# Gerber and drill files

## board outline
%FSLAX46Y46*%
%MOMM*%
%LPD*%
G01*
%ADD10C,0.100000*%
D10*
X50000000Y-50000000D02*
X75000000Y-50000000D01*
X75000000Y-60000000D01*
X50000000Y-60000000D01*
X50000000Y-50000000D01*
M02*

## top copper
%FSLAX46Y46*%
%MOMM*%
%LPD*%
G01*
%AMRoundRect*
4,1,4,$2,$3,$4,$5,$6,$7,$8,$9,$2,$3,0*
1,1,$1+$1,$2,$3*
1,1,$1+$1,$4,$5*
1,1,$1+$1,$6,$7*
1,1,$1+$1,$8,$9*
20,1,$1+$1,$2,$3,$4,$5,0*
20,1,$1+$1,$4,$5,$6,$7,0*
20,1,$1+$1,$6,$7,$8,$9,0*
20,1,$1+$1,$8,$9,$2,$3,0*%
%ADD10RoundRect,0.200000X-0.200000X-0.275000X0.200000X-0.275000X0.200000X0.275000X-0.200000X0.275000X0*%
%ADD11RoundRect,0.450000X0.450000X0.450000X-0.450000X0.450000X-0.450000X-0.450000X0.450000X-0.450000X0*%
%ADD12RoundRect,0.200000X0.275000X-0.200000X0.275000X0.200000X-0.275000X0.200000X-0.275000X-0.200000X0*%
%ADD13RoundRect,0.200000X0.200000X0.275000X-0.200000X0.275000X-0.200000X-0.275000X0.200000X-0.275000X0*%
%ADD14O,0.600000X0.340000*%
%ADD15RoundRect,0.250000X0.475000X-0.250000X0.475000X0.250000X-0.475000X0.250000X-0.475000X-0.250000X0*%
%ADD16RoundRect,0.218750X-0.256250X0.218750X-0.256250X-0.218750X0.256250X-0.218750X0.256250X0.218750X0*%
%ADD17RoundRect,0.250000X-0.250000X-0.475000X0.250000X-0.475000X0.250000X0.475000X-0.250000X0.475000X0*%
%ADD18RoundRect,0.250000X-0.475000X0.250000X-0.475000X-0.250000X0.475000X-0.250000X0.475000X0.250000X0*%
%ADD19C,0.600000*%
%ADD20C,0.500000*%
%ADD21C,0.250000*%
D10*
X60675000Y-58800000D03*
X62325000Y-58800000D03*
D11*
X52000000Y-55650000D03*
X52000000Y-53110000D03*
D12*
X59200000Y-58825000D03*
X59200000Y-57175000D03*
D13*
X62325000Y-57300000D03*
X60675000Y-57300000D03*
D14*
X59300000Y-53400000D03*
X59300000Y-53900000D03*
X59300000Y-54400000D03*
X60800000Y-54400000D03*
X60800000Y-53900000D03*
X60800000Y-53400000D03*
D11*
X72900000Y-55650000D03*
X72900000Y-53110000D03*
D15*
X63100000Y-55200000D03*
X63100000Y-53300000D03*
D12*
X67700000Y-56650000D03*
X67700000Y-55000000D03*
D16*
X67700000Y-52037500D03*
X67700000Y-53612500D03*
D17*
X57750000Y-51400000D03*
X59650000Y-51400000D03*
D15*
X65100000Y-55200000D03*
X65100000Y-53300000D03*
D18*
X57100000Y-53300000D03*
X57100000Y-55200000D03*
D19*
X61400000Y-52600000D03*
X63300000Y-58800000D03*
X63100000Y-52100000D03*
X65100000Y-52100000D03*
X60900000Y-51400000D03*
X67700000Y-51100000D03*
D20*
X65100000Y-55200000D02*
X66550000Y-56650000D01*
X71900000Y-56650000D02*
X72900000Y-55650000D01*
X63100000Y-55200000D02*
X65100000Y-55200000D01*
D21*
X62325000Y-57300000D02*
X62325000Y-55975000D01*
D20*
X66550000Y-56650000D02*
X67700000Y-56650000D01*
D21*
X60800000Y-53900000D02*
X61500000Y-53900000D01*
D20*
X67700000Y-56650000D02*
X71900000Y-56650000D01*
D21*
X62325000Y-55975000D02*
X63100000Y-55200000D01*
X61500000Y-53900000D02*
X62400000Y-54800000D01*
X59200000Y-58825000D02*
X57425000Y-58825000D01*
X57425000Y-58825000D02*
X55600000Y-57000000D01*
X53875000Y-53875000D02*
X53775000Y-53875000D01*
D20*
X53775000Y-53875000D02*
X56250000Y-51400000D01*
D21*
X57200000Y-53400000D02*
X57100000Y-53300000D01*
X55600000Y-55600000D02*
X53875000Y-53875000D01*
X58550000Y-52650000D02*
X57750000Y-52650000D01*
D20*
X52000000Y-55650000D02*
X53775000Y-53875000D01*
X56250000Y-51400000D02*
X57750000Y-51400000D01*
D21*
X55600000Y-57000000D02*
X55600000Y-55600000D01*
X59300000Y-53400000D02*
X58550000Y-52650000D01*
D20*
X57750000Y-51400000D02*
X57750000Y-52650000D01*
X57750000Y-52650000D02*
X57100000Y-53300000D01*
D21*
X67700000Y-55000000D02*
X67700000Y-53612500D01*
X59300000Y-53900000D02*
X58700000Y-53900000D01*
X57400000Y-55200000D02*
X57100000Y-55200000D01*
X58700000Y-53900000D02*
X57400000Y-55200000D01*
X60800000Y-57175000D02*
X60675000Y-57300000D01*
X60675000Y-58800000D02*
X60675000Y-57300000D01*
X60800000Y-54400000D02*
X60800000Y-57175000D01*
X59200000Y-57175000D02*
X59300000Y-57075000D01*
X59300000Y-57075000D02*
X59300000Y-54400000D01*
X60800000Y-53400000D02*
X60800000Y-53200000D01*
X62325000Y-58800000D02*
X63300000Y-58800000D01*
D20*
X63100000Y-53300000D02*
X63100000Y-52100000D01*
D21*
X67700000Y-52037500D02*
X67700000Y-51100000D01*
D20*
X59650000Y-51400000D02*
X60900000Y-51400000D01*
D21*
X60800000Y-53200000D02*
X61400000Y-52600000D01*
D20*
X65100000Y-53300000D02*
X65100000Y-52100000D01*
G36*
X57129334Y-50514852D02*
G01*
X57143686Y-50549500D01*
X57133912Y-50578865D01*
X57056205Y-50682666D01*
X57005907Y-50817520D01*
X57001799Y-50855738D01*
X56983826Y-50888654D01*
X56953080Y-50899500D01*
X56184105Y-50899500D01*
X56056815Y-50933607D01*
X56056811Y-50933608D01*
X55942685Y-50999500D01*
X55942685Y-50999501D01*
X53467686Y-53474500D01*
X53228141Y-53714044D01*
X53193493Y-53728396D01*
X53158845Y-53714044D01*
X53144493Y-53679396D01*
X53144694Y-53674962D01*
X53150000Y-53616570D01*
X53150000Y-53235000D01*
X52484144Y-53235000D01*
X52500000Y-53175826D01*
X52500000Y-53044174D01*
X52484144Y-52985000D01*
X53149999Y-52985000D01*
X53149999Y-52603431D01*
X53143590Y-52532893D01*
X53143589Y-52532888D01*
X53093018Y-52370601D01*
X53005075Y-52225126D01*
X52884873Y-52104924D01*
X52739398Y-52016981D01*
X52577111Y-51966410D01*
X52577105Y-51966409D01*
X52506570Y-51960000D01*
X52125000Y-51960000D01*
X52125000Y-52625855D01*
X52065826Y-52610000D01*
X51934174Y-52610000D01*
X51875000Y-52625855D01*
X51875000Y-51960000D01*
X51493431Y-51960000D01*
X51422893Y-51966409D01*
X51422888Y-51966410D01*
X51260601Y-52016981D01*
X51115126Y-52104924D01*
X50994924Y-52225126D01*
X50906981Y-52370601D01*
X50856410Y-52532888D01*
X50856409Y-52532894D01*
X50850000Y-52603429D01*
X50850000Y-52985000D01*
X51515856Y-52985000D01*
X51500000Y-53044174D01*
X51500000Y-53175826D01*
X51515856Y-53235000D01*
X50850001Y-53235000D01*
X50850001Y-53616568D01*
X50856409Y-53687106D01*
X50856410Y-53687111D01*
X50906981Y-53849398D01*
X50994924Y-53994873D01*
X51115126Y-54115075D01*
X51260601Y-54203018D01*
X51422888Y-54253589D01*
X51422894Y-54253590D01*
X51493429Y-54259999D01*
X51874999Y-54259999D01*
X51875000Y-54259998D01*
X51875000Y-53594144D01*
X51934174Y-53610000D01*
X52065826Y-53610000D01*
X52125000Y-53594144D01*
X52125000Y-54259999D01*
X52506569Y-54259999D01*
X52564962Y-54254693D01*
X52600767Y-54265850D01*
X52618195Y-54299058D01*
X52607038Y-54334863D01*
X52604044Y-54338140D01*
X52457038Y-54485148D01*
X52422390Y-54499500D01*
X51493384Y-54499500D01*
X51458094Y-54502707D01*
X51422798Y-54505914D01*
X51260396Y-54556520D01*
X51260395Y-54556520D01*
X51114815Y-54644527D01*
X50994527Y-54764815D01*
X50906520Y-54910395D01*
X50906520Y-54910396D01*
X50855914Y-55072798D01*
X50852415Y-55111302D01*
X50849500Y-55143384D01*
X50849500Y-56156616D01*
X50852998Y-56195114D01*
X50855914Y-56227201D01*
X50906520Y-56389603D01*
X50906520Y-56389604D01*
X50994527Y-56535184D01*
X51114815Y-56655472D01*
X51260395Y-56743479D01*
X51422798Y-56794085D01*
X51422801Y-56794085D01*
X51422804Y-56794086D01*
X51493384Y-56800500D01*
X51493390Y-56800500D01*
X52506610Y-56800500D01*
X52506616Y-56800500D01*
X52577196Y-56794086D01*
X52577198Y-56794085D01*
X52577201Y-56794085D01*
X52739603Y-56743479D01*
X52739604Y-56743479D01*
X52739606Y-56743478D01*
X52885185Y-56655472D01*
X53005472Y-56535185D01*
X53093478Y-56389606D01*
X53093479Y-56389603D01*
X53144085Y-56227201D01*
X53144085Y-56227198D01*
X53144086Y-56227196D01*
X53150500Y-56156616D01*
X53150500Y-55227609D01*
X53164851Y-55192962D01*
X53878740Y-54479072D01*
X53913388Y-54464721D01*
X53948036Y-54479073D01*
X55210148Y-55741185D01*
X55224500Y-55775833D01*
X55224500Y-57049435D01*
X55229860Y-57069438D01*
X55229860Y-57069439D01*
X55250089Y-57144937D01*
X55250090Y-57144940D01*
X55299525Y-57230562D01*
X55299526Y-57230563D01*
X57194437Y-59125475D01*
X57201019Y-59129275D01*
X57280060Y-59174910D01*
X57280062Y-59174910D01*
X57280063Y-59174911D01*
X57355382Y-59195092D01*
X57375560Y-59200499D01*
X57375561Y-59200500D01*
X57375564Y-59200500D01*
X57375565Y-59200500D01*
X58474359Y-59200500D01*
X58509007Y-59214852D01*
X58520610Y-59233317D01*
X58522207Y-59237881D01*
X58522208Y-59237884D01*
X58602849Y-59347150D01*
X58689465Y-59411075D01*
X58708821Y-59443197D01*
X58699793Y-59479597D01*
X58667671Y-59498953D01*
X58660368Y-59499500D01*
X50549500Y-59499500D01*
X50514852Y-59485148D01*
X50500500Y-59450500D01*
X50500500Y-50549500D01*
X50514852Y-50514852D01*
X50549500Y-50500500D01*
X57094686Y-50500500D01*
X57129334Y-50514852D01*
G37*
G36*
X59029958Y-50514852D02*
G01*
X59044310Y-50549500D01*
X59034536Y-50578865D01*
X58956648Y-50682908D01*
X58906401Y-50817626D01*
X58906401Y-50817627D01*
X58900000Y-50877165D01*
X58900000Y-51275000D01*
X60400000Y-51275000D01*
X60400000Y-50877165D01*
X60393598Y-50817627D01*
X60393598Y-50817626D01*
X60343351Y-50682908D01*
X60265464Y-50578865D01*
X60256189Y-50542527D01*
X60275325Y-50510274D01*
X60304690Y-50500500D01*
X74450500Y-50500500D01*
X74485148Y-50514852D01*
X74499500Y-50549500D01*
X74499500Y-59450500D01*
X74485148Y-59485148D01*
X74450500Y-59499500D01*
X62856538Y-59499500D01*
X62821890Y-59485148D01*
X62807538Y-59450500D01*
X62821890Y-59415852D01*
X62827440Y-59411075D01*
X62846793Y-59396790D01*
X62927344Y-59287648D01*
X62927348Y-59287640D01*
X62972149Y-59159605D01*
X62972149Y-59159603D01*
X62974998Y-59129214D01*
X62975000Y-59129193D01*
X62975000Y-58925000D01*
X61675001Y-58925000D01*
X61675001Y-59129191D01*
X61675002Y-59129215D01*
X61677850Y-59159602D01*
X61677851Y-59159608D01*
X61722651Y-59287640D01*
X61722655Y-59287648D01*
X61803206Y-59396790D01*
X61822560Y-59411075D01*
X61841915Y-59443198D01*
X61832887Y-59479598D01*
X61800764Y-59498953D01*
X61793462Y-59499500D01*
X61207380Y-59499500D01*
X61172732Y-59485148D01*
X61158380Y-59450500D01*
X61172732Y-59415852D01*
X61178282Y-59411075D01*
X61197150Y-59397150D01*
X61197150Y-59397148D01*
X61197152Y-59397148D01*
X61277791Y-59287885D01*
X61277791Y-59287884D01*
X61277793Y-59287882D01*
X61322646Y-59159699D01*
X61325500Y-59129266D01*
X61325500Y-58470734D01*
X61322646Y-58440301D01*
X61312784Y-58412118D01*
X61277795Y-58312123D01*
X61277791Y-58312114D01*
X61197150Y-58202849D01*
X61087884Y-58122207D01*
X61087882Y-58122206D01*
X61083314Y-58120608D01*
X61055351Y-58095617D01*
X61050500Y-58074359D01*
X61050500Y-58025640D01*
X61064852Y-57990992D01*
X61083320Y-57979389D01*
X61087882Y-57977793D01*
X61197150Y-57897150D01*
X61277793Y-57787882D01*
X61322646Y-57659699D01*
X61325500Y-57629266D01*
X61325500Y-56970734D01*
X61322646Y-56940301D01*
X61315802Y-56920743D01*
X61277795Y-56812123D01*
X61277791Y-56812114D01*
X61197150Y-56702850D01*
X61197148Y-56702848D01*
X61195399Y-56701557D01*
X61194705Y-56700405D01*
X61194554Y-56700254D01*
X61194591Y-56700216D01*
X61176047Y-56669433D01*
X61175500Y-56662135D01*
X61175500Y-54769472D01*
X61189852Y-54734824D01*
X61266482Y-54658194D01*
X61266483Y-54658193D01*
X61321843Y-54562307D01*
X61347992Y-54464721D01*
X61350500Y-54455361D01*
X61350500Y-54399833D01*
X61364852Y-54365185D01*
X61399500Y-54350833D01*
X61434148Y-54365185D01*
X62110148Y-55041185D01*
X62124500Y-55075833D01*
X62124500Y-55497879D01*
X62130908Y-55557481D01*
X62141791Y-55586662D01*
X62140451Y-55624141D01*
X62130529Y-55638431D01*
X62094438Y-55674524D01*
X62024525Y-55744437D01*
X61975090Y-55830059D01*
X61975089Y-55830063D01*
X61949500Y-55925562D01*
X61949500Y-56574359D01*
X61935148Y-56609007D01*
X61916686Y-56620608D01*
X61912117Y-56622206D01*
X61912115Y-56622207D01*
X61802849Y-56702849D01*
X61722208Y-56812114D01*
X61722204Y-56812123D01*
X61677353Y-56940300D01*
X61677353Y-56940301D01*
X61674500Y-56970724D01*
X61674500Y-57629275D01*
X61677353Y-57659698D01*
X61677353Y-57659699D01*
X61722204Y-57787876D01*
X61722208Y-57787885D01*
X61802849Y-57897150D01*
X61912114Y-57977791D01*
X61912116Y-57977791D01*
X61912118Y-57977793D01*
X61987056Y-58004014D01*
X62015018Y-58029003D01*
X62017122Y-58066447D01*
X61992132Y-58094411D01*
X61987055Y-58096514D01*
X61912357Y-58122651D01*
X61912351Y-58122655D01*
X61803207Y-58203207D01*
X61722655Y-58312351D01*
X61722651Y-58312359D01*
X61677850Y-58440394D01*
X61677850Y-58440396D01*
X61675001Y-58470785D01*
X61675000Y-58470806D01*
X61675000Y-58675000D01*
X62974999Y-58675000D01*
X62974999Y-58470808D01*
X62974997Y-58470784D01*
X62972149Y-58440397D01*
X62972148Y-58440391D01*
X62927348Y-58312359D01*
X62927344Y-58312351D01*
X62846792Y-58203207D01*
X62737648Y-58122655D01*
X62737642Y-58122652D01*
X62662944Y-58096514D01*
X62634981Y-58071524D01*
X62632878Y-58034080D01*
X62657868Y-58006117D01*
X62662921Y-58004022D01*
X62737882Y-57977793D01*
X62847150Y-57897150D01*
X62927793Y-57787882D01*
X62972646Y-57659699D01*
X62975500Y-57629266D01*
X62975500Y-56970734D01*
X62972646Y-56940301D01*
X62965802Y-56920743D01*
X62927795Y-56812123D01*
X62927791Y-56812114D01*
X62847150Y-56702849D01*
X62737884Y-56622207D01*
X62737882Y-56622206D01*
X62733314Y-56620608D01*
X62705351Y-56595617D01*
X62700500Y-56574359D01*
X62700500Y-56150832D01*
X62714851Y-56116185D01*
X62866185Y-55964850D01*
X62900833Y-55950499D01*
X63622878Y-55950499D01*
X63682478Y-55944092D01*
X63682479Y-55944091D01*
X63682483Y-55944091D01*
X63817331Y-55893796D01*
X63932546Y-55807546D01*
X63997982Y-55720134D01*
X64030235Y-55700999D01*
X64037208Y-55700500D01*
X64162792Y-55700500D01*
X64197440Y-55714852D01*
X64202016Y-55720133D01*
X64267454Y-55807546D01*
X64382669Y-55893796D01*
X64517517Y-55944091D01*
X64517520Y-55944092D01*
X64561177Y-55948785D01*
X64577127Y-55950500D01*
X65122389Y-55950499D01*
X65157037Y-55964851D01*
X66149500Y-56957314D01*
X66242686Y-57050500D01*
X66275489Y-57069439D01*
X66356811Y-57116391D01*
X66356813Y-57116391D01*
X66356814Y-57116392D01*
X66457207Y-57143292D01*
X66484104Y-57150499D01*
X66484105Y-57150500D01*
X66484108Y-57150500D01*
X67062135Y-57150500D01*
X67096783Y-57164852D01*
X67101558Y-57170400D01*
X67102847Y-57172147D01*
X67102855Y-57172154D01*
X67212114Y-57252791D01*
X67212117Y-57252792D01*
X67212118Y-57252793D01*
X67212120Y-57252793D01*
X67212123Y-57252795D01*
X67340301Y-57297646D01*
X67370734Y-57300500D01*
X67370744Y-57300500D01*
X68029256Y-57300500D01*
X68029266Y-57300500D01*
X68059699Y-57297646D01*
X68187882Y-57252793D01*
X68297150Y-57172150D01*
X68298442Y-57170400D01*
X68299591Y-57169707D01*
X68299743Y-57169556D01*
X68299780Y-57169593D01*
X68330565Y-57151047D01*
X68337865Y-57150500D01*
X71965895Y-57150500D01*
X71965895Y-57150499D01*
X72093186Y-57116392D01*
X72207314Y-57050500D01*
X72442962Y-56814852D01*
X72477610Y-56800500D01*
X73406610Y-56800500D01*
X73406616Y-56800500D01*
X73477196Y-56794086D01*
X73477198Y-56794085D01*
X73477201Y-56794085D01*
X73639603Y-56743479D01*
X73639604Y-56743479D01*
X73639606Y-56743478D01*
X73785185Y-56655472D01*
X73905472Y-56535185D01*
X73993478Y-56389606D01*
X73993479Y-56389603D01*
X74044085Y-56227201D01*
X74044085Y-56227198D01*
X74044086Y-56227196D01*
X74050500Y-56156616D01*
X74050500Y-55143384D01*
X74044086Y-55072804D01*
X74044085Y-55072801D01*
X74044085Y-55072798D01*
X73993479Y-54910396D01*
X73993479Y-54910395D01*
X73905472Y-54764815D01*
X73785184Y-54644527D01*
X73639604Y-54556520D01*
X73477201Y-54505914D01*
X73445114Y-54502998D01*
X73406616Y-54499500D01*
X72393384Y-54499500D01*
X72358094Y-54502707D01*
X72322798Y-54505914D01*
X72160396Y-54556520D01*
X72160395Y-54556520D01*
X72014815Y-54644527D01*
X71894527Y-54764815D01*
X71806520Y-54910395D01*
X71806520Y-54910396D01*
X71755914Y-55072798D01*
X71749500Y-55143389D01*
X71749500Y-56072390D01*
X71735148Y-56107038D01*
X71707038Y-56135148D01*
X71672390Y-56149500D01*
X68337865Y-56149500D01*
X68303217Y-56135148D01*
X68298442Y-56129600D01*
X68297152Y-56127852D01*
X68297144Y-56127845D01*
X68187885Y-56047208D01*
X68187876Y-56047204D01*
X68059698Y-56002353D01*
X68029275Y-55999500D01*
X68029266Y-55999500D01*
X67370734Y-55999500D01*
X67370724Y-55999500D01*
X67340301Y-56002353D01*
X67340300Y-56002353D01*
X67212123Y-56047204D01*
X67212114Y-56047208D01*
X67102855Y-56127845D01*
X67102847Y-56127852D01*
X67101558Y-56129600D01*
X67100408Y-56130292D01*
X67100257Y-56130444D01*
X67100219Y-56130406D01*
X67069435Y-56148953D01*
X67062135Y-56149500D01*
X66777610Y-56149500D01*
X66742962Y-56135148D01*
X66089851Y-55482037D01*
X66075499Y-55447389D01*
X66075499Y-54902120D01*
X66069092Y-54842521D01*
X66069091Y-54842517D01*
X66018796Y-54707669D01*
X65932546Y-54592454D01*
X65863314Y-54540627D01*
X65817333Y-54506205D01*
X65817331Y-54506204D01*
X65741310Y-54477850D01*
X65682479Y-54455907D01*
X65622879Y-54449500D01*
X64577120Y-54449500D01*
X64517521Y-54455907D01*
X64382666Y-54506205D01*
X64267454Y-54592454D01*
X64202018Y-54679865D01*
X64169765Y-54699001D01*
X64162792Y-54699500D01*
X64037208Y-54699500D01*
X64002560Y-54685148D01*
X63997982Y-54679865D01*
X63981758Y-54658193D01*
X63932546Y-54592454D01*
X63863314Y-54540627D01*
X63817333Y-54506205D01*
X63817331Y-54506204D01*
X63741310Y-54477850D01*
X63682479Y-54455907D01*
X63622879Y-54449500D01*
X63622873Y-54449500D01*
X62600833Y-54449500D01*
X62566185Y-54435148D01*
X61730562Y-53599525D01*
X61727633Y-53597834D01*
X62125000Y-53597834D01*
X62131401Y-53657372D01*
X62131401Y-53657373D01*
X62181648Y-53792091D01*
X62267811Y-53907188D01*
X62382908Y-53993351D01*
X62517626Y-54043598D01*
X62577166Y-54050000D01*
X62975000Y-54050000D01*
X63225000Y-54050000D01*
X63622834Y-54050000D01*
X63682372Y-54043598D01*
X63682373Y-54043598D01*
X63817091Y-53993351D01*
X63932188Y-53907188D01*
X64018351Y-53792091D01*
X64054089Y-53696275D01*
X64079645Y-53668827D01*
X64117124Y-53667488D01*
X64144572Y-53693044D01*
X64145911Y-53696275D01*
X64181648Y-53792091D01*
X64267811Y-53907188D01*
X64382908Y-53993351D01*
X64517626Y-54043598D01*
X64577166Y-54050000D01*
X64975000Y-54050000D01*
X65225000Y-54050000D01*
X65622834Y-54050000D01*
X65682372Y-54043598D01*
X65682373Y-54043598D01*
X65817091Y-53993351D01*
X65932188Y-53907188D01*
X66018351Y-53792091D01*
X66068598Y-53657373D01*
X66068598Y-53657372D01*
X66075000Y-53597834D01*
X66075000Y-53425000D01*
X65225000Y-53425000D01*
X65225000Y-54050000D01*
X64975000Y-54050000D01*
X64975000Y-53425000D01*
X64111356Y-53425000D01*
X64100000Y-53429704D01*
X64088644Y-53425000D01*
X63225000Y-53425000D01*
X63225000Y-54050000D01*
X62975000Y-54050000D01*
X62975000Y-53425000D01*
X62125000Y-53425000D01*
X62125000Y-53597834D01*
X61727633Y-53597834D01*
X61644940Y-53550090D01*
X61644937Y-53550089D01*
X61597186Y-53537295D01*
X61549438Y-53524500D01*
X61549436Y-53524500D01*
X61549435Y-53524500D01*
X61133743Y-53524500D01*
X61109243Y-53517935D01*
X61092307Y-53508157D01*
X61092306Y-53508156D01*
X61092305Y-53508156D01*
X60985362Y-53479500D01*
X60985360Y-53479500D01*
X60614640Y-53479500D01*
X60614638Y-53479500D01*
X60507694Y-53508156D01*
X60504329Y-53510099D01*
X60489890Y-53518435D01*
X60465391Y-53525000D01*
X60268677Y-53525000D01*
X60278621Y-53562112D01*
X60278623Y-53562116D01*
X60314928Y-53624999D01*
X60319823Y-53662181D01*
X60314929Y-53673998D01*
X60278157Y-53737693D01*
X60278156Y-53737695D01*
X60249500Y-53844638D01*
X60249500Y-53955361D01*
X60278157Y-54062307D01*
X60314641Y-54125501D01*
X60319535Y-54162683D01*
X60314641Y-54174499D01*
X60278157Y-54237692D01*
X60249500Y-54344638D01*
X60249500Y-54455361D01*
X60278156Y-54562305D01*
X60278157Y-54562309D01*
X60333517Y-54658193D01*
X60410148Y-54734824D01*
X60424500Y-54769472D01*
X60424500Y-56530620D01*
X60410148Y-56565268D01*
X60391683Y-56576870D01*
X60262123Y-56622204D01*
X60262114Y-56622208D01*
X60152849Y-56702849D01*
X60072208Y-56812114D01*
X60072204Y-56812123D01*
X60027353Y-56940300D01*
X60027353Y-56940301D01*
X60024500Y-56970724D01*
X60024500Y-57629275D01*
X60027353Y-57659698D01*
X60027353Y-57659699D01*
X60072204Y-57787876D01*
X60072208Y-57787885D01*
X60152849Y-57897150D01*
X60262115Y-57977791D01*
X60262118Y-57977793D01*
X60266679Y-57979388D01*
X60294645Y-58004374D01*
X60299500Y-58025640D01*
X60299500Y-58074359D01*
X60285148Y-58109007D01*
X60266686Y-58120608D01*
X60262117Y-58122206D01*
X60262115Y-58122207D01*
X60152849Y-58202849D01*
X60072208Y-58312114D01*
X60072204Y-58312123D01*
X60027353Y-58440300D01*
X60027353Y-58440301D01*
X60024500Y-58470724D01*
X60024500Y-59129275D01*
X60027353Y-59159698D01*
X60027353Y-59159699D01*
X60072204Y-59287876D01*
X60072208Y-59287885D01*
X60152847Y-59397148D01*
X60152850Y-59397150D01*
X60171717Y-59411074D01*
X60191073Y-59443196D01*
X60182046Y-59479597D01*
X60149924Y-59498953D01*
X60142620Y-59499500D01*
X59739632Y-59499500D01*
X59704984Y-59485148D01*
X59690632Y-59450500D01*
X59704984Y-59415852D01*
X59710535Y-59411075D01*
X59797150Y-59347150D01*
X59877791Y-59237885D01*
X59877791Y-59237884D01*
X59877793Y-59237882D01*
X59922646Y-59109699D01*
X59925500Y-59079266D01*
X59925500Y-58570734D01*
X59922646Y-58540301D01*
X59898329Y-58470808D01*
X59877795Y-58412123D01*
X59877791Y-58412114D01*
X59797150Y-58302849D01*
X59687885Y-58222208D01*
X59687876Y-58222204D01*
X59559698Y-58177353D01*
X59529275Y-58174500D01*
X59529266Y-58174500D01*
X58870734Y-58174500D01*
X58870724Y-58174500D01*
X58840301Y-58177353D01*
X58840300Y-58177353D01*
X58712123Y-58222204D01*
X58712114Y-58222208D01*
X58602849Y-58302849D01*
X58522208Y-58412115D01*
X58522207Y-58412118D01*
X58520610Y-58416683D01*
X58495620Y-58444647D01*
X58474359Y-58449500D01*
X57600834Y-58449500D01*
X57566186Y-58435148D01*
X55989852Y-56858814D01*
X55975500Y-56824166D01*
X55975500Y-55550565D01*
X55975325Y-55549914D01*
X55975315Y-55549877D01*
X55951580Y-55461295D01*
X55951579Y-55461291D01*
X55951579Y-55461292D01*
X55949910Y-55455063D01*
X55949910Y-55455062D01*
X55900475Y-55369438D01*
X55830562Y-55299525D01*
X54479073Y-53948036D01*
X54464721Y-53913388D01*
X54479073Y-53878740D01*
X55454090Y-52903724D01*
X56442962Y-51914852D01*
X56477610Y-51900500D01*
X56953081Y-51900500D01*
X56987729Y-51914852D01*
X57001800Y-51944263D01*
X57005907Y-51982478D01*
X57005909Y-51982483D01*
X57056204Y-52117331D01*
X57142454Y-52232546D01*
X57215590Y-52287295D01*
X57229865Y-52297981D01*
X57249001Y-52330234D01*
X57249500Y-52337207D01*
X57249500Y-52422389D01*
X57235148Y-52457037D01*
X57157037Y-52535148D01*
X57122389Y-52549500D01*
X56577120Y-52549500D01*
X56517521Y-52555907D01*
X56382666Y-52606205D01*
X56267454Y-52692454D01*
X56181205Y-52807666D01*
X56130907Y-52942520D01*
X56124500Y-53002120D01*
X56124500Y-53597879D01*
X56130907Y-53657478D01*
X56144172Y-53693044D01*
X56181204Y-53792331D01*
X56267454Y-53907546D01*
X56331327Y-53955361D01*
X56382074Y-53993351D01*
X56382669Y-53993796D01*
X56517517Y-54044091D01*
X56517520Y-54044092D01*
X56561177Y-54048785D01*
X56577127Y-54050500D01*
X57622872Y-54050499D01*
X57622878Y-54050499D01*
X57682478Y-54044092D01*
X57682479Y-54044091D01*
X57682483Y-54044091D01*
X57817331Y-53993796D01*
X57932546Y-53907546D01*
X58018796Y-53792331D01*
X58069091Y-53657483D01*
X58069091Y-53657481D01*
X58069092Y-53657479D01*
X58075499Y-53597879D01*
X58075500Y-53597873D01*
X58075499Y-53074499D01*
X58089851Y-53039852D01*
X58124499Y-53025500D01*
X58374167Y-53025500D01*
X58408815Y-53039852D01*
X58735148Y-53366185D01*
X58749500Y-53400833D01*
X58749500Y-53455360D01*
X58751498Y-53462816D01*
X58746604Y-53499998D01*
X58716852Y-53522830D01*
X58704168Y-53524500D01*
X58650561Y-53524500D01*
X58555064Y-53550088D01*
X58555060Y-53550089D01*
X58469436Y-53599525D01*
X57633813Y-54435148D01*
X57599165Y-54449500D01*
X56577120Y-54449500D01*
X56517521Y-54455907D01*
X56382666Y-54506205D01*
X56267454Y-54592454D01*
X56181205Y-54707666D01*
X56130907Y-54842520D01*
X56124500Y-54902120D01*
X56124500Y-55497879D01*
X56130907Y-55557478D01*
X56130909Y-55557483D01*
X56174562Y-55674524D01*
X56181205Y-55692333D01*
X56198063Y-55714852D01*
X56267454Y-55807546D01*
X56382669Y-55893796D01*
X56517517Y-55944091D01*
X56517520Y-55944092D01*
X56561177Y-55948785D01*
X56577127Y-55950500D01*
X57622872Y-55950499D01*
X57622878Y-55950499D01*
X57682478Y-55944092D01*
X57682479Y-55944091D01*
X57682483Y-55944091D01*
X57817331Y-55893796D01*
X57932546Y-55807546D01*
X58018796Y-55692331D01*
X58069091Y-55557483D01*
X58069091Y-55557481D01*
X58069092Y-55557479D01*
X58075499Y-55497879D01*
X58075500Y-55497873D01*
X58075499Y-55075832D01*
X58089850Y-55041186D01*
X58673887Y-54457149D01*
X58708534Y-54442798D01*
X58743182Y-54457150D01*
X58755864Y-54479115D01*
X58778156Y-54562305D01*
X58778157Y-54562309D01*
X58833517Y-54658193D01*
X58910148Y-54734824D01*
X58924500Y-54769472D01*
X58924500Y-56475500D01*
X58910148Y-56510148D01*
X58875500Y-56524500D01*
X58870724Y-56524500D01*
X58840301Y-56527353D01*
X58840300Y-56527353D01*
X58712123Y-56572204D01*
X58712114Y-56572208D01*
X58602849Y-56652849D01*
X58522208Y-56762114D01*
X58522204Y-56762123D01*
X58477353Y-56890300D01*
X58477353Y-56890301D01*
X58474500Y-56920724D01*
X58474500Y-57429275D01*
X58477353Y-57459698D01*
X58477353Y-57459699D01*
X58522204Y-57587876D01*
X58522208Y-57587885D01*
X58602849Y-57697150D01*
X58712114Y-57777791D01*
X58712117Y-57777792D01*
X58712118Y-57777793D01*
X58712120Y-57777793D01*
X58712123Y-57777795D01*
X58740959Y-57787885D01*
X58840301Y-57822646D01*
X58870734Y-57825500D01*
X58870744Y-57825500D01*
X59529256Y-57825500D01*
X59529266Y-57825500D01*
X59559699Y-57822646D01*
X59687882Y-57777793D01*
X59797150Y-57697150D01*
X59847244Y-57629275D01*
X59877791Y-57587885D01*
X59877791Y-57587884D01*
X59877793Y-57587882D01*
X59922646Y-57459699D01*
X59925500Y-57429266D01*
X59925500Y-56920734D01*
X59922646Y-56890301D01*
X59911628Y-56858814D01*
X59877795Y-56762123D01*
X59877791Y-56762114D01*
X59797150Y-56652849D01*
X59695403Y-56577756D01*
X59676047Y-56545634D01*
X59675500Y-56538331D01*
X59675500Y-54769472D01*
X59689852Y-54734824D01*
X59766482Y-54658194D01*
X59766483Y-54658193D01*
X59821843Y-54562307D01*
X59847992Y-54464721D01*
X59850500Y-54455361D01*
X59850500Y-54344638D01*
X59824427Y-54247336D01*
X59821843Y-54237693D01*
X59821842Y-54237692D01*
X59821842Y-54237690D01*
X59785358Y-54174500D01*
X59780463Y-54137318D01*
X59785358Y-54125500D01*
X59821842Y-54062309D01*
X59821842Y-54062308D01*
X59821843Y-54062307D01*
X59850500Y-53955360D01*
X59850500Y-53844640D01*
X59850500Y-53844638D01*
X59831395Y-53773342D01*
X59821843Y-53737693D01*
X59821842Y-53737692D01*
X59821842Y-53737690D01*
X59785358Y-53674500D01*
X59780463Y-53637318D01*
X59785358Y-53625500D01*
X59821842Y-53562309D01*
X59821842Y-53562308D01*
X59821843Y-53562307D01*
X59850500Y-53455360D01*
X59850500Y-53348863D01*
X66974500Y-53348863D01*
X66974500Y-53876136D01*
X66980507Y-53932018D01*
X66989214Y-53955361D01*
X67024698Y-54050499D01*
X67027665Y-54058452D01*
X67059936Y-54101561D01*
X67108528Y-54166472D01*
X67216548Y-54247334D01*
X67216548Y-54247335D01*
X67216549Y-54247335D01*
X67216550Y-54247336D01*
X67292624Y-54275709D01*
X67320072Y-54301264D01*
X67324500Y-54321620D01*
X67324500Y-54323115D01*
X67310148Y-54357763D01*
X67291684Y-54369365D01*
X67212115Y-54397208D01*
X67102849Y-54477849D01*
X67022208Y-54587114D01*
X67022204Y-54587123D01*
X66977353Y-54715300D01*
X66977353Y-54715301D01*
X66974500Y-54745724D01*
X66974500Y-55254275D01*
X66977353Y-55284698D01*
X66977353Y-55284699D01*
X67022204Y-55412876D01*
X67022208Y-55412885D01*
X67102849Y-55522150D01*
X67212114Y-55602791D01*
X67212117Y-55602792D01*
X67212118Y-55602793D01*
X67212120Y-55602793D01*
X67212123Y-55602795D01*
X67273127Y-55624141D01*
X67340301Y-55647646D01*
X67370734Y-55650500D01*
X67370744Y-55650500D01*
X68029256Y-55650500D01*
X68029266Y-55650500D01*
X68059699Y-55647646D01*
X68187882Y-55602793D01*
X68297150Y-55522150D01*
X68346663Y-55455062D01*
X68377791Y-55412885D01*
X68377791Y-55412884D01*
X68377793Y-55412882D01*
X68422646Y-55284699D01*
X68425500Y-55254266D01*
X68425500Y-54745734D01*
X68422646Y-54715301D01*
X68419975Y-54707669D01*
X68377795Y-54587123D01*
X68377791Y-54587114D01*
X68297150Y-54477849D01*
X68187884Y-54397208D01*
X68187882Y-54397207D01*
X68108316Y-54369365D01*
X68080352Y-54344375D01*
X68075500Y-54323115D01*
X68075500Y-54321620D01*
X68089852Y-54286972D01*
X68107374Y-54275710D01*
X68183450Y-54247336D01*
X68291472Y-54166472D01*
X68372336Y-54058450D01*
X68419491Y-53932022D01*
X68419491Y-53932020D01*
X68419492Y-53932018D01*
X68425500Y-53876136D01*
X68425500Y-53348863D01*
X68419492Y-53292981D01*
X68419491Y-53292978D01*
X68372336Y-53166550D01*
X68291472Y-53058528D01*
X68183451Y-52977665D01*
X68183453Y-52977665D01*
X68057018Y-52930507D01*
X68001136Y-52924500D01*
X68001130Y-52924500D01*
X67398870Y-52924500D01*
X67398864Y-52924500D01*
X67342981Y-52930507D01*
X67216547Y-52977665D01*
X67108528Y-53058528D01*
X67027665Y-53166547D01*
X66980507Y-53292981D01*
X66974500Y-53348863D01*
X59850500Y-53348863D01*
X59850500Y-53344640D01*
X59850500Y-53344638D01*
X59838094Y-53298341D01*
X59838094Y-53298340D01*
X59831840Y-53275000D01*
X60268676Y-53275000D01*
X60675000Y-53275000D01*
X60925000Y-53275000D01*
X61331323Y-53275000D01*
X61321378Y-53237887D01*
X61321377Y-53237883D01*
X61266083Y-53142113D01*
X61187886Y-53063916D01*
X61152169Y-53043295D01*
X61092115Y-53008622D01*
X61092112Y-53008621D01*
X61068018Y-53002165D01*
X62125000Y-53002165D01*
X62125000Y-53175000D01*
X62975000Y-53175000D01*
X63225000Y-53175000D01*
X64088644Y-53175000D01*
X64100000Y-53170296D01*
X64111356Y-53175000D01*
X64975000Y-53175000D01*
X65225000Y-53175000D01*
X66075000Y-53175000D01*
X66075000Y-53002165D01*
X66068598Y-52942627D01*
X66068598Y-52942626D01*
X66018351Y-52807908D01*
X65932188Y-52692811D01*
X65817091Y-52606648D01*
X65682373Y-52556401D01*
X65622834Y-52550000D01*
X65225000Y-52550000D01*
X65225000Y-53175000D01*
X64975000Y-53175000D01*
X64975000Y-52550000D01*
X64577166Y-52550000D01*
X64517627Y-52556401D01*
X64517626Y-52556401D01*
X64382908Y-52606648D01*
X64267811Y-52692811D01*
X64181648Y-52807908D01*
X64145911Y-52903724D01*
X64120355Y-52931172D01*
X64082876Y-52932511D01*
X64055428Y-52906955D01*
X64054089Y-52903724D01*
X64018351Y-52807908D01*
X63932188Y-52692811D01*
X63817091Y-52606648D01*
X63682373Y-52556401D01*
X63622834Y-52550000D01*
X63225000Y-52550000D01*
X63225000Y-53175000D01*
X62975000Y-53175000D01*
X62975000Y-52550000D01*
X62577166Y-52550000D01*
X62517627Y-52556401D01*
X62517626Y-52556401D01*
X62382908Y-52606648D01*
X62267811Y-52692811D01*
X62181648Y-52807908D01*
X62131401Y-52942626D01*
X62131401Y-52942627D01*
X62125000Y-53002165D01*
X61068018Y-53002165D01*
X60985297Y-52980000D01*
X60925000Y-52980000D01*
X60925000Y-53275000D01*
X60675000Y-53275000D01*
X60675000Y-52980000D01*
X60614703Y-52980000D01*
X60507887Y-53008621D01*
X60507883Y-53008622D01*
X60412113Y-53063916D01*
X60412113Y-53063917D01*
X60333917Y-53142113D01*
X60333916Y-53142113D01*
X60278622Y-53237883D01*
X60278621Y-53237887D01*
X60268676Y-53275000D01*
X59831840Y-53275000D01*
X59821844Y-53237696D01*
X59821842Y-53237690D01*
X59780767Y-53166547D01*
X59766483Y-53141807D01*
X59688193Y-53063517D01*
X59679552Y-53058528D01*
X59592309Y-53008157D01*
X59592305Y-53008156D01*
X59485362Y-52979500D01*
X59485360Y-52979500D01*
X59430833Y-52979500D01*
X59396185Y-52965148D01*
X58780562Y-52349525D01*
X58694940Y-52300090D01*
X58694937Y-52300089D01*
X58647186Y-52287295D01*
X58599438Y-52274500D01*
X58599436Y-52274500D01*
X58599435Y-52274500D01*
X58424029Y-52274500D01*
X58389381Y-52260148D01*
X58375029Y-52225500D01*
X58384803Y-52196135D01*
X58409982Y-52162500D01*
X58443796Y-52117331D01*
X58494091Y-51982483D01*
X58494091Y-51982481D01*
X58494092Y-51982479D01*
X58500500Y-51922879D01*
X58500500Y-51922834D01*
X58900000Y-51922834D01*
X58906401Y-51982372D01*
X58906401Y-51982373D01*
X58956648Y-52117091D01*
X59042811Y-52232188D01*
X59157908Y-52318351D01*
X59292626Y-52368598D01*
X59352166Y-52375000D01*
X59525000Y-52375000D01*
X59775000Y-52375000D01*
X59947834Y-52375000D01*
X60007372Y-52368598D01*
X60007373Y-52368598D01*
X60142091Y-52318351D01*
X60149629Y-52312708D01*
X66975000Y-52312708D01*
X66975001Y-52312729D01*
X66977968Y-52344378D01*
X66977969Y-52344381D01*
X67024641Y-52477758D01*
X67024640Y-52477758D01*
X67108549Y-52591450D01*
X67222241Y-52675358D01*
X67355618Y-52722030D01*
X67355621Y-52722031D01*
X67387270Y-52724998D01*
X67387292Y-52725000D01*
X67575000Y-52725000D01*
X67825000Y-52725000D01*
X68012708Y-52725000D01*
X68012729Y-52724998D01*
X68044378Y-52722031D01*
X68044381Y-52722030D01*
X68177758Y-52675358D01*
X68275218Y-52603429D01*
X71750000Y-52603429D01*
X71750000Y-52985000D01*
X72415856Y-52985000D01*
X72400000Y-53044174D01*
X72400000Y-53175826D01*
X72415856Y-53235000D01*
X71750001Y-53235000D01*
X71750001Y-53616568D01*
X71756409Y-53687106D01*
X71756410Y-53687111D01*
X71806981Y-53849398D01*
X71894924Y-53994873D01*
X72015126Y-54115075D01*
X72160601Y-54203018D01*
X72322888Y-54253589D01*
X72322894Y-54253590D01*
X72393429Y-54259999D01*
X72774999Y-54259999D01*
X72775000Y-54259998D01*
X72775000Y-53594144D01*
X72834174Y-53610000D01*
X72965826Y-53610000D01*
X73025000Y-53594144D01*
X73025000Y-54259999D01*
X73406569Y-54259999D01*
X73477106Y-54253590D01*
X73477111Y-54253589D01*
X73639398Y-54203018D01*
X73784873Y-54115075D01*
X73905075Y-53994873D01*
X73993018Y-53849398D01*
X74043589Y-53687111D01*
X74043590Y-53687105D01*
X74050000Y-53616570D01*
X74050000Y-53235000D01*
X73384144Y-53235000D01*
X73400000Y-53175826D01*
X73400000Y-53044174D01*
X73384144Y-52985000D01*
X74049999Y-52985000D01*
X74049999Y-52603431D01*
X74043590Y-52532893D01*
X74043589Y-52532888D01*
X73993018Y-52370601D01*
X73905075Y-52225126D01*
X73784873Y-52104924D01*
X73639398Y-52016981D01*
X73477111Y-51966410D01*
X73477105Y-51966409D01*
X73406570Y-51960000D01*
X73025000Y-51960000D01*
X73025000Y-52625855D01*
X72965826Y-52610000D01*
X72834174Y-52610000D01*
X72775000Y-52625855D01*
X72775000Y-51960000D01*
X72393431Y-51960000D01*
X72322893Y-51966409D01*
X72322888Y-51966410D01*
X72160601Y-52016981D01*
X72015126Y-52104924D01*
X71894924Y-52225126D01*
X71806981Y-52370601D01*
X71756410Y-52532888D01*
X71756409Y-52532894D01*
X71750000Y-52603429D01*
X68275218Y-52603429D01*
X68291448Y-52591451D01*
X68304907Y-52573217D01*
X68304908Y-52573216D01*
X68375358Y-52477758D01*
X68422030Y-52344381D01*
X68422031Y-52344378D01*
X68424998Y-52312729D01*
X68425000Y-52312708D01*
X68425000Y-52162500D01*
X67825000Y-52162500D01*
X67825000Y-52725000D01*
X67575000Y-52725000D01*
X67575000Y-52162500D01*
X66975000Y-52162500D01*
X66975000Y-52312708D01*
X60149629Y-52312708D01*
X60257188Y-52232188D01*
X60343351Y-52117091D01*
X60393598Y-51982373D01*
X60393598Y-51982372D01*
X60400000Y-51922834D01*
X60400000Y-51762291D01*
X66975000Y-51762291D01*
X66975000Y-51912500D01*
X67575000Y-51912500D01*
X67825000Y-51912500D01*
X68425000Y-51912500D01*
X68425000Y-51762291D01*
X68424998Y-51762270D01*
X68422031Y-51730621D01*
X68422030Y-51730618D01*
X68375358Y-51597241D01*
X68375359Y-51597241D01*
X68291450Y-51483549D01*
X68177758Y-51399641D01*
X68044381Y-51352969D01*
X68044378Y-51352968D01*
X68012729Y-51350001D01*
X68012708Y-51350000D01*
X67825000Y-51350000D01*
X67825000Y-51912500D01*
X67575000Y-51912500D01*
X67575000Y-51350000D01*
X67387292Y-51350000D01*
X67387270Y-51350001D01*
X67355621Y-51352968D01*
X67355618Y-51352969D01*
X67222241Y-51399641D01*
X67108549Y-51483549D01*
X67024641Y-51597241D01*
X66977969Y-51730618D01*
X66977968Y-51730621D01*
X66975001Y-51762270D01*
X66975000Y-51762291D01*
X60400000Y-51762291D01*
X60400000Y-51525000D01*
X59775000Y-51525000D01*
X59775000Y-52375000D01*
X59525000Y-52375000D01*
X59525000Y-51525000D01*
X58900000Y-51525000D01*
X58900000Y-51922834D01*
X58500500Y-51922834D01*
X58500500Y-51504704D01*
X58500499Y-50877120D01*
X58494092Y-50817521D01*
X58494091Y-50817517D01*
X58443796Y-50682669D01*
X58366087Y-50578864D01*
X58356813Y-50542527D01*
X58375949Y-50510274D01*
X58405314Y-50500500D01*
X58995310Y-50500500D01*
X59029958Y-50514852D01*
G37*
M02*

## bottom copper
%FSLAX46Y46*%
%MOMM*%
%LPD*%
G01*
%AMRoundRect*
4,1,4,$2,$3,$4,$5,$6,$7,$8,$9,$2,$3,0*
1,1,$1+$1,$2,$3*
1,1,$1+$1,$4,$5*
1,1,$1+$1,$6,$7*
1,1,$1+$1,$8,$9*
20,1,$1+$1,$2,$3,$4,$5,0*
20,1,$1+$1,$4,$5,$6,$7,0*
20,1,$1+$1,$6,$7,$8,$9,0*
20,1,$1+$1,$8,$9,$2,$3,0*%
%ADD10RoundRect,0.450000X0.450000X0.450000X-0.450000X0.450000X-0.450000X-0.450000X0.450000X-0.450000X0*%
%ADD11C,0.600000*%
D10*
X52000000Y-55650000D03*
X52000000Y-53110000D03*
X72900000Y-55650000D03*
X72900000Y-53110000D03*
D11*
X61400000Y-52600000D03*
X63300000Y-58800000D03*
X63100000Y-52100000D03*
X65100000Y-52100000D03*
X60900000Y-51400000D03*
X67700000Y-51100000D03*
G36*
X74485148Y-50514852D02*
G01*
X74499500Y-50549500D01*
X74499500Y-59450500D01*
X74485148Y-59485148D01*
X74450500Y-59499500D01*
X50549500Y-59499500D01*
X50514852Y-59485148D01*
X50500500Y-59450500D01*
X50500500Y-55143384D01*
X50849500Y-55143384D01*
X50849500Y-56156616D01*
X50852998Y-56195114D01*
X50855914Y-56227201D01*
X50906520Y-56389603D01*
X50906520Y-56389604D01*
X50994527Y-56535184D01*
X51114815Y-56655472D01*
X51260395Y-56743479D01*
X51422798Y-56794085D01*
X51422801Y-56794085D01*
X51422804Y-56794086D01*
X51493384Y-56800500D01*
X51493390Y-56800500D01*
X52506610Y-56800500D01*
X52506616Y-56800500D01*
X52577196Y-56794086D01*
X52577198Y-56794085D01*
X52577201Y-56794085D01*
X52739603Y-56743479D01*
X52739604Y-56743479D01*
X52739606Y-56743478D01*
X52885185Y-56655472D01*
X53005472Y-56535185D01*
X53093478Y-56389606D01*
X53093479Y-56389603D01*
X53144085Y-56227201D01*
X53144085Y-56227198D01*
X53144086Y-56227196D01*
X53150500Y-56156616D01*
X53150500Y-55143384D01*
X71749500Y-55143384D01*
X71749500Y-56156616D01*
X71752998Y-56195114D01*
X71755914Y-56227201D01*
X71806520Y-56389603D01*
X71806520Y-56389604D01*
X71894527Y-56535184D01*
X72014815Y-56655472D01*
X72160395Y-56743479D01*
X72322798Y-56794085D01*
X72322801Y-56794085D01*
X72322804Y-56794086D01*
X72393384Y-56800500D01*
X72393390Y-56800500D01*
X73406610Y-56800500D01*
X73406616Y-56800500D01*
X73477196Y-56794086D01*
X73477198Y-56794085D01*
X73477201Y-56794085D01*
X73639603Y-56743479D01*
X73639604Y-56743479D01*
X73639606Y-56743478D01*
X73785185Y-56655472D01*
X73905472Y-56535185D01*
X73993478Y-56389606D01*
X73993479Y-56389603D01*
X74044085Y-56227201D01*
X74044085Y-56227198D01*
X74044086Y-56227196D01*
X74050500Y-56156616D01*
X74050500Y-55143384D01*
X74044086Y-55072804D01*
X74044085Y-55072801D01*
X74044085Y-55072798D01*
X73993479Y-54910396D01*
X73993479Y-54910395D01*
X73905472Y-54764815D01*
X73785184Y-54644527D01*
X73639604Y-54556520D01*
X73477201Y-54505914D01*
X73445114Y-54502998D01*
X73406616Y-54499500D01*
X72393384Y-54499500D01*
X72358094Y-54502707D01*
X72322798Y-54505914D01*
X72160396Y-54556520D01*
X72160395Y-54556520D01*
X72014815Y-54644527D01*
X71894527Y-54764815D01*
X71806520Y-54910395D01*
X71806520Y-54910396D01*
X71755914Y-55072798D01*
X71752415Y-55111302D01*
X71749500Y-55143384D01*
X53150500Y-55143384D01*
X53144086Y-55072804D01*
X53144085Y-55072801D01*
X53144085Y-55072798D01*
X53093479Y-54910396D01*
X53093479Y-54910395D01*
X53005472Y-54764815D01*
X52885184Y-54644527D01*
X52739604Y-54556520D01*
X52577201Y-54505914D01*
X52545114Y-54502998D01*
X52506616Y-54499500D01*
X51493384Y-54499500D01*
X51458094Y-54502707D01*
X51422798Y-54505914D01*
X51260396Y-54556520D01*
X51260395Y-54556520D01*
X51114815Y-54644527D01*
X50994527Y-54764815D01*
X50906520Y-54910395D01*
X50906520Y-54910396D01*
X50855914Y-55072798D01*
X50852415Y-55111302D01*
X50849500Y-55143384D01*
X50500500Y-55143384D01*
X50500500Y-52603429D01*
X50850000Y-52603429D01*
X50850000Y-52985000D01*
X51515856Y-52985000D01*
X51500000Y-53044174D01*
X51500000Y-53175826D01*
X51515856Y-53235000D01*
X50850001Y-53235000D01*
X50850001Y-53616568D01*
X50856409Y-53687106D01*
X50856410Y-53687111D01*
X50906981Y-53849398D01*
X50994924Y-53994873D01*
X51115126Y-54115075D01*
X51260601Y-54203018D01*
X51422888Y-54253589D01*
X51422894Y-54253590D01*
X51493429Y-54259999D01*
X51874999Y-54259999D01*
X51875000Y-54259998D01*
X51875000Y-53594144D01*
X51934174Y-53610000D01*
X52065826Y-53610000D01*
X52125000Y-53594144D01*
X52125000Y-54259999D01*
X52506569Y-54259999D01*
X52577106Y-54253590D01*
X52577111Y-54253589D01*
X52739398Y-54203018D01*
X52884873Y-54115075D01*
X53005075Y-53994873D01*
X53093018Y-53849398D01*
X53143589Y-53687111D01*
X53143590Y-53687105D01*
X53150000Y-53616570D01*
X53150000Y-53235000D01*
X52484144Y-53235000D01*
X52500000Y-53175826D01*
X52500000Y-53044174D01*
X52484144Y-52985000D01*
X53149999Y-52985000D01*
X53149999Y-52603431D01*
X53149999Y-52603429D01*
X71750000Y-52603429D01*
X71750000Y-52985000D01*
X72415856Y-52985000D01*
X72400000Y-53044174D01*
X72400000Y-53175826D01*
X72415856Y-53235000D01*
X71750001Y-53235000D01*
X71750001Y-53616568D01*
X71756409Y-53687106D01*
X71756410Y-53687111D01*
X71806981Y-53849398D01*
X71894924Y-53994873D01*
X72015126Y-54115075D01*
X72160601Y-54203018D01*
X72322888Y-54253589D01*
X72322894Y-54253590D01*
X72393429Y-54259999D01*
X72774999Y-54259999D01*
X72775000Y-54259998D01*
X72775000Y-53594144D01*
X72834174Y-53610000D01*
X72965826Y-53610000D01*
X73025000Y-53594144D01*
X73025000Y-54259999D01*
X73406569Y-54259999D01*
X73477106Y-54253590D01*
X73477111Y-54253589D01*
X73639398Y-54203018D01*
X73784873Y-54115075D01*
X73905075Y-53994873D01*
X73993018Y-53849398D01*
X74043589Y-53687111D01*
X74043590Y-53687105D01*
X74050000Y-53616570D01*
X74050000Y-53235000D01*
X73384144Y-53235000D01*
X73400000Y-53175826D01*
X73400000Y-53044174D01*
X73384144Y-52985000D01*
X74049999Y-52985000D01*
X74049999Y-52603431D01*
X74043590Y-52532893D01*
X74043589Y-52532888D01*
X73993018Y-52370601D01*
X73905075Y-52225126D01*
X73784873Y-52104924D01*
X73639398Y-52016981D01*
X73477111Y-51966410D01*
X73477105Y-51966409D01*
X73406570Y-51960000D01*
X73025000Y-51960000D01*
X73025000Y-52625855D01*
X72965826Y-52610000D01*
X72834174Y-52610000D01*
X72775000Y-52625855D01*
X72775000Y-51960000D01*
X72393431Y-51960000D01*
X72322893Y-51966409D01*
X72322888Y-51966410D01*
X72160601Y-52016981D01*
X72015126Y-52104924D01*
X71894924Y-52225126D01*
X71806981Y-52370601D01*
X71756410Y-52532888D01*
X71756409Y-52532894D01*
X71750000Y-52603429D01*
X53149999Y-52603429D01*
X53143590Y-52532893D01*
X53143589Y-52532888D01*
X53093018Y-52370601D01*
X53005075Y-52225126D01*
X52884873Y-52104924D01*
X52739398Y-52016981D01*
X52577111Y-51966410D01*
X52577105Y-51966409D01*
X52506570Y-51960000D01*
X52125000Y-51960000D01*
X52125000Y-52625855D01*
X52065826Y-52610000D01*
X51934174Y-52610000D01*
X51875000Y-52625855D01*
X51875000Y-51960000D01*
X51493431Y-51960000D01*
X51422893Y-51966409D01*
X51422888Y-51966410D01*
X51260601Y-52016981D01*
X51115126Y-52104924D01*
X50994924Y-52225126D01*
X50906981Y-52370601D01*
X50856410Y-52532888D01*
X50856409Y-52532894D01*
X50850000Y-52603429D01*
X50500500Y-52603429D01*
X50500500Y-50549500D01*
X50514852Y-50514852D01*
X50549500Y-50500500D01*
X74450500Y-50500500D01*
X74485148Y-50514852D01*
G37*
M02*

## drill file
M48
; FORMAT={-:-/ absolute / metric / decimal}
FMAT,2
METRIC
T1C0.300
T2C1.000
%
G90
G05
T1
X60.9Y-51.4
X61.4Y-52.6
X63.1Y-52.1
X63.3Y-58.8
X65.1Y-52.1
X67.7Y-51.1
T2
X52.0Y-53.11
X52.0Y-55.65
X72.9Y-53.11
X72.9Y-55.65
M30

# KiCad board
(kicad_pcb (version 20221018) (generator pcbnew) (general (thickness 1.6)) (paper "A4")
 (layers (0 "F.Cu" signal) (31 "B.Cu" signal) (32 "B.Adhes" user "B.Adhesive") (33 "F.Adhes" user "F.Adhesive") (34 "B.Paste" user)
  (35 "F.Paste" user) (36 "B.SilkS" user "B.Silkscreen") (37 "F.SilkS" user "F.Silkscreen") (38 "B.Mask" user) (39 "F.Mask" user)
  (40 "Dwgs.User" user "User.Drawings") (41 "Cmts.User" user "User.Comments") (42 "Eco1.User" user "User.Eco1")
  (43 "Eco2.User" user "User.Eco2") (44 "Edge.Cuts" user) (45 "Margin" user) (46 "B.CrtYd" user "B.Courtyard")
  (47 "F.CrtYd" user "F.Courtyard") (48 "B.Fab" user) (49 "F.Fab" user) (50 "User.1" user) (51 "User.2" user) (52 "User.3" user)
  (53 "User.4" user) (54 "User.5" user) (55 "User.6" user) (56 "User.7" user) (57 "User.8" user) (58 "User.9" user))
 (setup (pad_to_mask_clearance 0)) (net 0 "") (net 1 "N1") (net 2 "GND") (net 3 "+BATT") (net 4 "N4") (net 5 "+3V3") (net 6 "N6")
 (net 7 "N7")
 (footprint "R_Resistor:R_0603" (layer "F.Cu") (at 61.5 58.8)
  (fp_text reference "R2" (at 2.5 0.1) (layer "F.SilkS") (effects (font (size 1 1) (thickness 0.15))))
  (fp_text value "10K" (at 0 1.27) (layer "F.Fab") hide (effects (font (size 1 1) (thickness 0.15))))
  (pad "1" smd roundrect (at -0.825 0) (size 0.8 0.95) (layers "F.Cu" "F.Paste" "F.Mask") (roundrect_rratio 0.25) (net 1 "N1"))
  (pad "2" smd roundrect (at 0.825 0) (size 0.8 0.95) (layers "F.Cu" "F.Paste" "F.Mask") (roundrect_rratio 0.25) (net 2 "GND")))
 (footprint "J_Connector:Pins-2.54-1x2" (layer "F.Cu") (at 52 55.65 180)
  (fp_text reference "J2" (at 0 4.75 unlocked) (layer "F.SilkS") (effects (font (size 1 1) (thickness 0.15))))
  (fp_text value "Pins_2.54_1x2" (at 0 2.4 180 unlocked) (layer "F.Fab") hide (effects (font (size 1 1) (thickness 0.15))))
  (pad "1" thru_hole roundrect (at 0 0 180) (size 1.8 1.8) (drill 1) (layers "*.Cu" "*.Mask") (roundrect_rratio 0.25) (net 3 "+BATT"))
  (pad "2" thru_hole roundrect (at 0 2.54 180) (size 1.8 1.8) (drill 1) (layers "*.Cu" "*.Mask") (roundrect_rratio 0.25) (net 2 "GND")))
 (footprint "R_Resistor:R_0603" (layer "F.Cu") (at 59.2 58 90)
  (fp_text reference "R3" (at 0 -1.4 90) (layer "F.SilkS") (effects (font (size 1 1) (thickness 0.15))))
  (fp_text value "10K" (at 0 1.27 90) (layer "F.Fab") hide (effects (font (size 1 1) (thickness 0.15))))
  (pad "1" smd roundrect (at -0.825 0 90) (size 0.8 0.95) (layers "F.Cu" "F.Paste" "F.Mask") (roundrect_rratio 0.25) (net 3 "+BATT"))
  (pad "2" smd roundrect (at 0.825 0 90) (size 0.8 0.95) (layers "F.Cu" "F.Paste" "F.Mask") (roundrect_rratio 0.25) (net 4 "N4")))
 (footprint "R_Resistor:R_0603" (layer "F.Cu") (at 61.5 57.3 180)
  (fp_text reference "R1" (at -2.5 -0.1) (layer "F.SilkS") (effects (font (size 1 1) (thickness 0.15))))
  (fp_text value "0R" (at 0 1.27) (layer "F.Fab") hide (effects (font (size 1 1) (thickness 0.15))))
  (pad "1" smd roundrect (at -0.825 0 180) (size 0.8 0.95) (layers "F.Cu" "F.Paste" "F.Mask") (roundrect_rratio 0.25) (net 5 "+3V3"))
  (pad "2" smd roundrect (at 0.825 0 180) (size 0.8 0.95) (layers "F.Cu" "F.Paste" "F.Mask") (roundrect_rratio 0.25) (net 1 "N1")))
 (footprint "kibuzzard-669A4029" (layer "F.Cu") (at 52.8 58.8)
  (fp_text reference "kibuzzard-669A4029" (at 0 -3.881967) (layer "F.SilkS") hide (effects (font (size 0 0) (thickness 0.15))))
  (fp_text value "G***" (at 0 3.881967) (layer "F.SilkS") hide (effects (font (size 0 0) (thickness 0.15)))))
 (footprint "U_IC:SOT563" (layer "F.Cu") (at 60.05 53.9)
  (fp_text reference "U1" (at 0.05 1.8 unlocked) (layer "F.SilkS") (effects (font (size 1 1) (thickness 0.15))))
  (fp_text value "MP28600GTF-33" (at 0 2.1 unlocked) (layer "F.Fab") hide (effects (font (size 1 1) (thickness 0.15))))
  (pad "1" smd oval (at -0.75 -0.5) (size 0.6 0.34) (layers "F.Cu" "F.Paste" "F.Mask") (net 3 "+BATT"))
  (pad "2" smd oval (at -0.75 0) (size 0.6 0.34) (layers "F.Cu" "F.Paste" "F.Mask") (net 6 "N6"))
  (pad "3" smd oval (at -0.75 0.5) (size 0.6 0.34) (layers "F.Cu" "F.Paste" "F.Mask") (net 4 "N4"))
  (pad "4" smd oval (at 0.75 0.5) (size 0.6 0.34) (layers "F.Cu" "F.Paste" "F.Mask") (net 1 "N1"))
  (pad "5" smd oval (at 0.75 0) (size 0.6 0.34) (layers "F.Cu" "F.Paste" "F.Mask") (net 5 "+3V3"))
  (pad "6" smd oval (at 0.75 -0.5) (size 0.6 0.34) (layers "F.Cu" "F.Paste" "F.Mask") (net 2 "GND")))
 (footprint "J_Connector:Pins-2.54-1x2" (layer "F.Cu") (at 72.9 55.65 180)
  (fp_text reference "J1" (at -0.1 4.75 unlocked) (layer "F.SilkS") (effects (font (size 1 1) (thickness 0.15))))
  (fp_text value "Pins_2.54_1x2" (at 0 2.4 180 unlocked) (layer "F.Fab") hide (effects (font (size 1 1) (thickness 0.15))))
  (pad "1" thru_hole roundrect (at 0 0 180) (size 1.8 1.8) (drill 1) (layers "*.Cu" "*.Mask") (roundrect_rratio 0.25) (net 5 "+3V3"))
  (pad "2" thru_hole roundrect (at 0 2.54 180) (size 1.8 1.8) (drill 1) (layers "*.Cu" "*.Mask") (roundrect_rratio 0.25) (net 2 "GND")))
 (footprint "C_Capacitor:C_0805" (layer "F.Cu") (at 63.1 54.25 90)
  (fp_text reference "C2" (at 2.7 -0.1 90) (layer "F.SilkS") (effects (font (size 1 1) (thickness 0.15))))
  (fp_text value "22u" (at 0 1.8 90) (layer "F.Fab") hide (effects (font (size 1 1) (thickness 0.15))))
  (pad "1" smd roundrect (at -0.95 0 90) (size 1 1.45) (layers "F.Cu" "F.Paste" "F.Mask") (roundrect_rratio 0.25) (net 5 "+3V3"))
  (pad "2" smd roundrect (at 0.95 0 90) (size 1 1.45) (layers "F.Cu" "F.Paste" "F.Mask") (roundrect_rratio 0.25) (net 2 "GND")))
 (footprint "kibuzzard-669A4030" (layer "F.Cu") (at 72.5 58.8)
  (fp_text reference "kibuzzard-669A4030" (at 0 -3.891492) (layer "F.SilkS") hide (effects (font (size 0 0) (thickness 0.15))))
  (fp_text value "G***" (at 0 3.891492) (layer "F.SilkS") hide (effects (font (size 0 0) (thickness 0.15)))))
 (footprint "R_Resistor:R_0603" (layer "F.Cu") (at 67.7 55.825 90)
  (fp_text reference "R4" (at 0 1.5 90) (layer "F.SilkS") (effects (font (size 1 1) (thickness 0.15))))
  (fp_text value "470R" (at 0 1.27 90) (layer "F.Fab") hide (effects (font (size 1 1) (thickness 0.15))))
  (pad "1" smd roundrect (at -0.825 0 90) (size 0.8 0.95) (layers "F.Cu" "F.Paste" "F.Mask") (roundrect_rratio 0.25) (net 5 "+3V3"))
  (pad "2" smd roundrect (at 0.825 0 90) (size 0.8 0.95) (layers "F.Cu" "F.Paste" "F.Mask") (roundrect_rratio 0.25) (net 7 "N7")))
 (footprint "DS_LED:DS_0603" (layer "F.Cu") (at 67.7 52.825 -90)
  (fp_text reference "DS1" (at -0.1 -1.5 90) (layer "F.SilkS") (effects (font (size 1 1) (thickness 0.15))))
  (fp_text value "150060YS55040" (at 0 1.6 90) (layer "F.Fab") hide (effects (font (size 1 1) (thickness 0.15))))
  (pad "1" smd roundrect (at -0.7875 0 270) (size 0.875 0.95) (layers "F.Cu" "F.Paste" "F.Mask") (roundrect_rratio 0.25) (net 2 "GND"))
  (pad "2" smd roundrect (at 0.7875 0 270) (size 0.875 0.95) (layers "F.Cu" "F.Paste" "F.Mask") (roundrect_rratio 0.25) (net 7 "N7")))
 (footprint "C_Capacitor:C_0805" (layer "F.Cu") (at 58.7 51.4)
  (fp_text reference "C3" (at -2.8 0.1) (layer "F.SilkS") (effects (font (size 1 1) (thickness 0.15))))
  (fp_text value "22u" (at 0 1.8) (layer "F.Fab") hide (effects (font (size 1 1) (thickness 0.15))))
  (pad "1" smd roundrect (at -0.95 0) (size 1 1.45) (layers "F.Cu" "F.Paste" "F.Mask") (roundrect_rratio 0.25) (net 3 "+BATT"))
  (pad "2" smd roundrect (at 0.95 0) (size 1 1.45) (layers "F.Cu" "F.Paste" "F.Mask") (roundrect_rratio 0.25) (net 2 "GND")))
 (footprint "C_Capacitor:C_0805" (layer "F.Cu") (at 65.1 54.25 90)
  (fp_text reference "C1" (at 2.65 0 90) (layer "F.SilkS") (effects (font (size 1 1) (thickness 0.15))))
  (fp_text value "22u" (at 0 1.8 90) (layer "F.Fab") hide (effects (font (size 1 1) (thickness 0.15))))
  (pad "1" smd roundrect (at -0.95 0 90) (size 1 1.45) (layers "F.Cu" "F.Paste" "F.Mask") (roundrect_rratio 0.25) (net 5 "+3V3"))
  (pad "2" smd roundrect (at 0.95 0 90) (size 1 1.45) (layers "F.Cu" "F.Paste" "F.Mask") (roundrect_rratio 0.25) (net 2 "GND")))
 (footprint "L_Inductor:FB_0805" (layer "F.Cu") (at 57.1 54.25 -90)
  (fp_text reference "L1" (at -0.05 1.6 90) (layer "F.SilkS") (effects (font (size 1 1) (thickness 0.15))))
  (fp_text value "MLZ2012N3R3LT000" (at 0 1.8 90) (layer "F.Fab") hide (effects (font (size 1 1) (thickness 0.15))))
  (pad "1" smd roundrect (at -0.95 0 270) (size 1 1.45) (layers "F.Cu" "F.Paste" "F.Mask") (roundrect_rratio 0.25) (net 3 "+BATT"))
  (pad "2" smd roundrect (at 0.95 0 270) (size 1 1.45) (layers "F.Cu" "F.Paste" "F.Mask") (roundrect_rratio 0.25) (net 6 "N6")))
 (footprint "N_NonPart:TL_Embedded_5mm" (layer "B.Cu") (at 59.8 56.2 180)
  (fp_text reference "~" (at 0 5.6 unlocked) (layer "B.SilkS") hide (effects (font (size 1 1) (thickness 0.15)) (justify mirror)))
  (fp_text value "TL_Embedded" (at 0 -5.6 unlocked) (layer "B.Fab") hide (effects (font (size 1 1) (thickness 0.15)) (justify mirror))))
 (gr_rect (start 50 50) (end 75 60) (stroke (width 0.1) (type default)) (fill none) (layer "Edge.Cuts"))
 (segment (start 65.1 55.2) (end 66.55 56.65) (width 0.5) (layer "F.Cu") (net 5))
 (segment (start 71.9 56.65) (end 72.9 55.65) (width 0.5) (layer "F.Cu") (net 5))
 (segment (start 63.1 55.2) (end 65.1 55.2) (width 0.5) (layer "F.Cu") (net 5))
 (segment (start 62.325 57.3) (end 62.325 55.975) (width 0.25) (layer "F.Cu") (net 5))
 (segment (start 66.55 56.65) (end 67.7 56.65) (width 0.5) (layer "F.Cu") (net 5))
 (segment (start 60.8 53.9) (end 61.5 53.9) (width 0.25) (layer "F.Cu") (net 5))
 (segment (start 67.7 56.65) (end 71.9 56.65) (width 0.5) (layer "F.Cu") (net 5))
 (segment (start 62.325 55.975) (end 63.1 55.2) (width 0.25) (layer "F.Cu") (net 5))
 (segment (start 61.5 53.9) (end 62.4 54.8) (width 0.25) (layer "F.Cu") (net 5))
 (segment (start 59.2 58.825) (end 57.425 58.825) (width 0.25) (layer "F.Cu") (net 3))
 (segment (start 57.425 58.825) (end 55.6 57) (width 0.25) (layer "F.Cu") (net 3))
 (segment (start 53.875 53.875) (end 53.775 53.875) (width 0.25) (layer "F.Cu") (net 3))
 (segment (start 53.775 53.875) (end 56.25 51.4) (width 0.5) (layer "F.Cu") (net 3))
 (segment (start 57.2 53.4) (end 57.1 53.3) (width 0.25) (layer "F.Cu") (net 3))
 (segment (start 55.6 55.6) (end 53.875 53.875) (width 0.25) (layer "F.Cu") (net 3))
 (segment (start 58.55 52.65) (end 57.75 52.65) (width 0.25) (layer "F.Cu") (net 3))
 (segment (start 52 55.65) (end 53.775 53.875) (width 0.5) (layer "F.Cu") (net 3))
 (segment (start 56.25 51.4) (end 57.75 51.4) (width 0.5) (layer "F.Cu") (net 3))
 (segment (start 55.6 57) (end 55.6 55.6) (width 0.25) (layer "F.Cu") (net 3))
 (segment (start 59.3 53.4) (end 58.55 52.65) (width 0.25) (layer "F.Cu") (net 3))
 (segment (start 57.75 51.4) (end 57.75 52.65) (width 0.5) (layer "F.Cu") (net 3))
 (segment (start 57.75 52.65) (end 57.1 53.3) (width 0.5) (layer "F.Cu") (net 3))
 (segment (start 67.7 55) (end 67.7 53.6125) (width 0.25) (layer "F.Cu") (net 7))
 (segment (start 59.3 53.9) (end 58.7 53.9) (width 0.25) (layer "F.Cu") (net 6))
 (segment (start 57.4 55.2) (end 57.1 55.2) (width 0.25) (layer "F.Cu") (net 6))
 (segment (start 58.7 53.9) (end 57.4 55.2) (width 0.25) (layer "F.Cu") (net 6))
 (segment (start 60.8 57.175) (end 60.675 57.3) (width 0.25) (layer "F.Cu") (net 1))
 (segment (start 60.675 58.8) (end 60.675 57.3) (width 0.25) (layer "F.Cu") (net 1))
 (segment (start 60.8 54.4) (end 60.8 57.175) (width 0.25) (layer "F.Cu") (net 1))
 (segment (start 59.2 57.175) (end 59.3 57.075) (width 0.25) (layer "F.Cu") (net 4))
 (segment (start 59.3 57.075) (end 59.3 54.4) (width 0.25) (layer "F.Cu") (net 4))
 (segment (start 60.8 53.4) (end 60.8 53.2) (width 0.25) (layer "F.Cu") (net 2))
 (segment (start 62.325 58.8) (end 63.3 58.8) (width 0.25) (layer "F.Cu") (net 2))
 (segment (start 63.1 53.3) (end 63.1 52.1) (width 0.5) (layer "F.Cu") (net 2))
 (segment (start 67.7 52.0375) (end 67.7 51.1) (width 0.25) (layer "F.Cu") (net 2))
 (segment (start 59.65 51.4) (end 60.9 51.4) (width 0.5) (layer "F.Cu") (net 2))
 (segment (start 60.8 53.2) (end 61.4 52.6) (width 0.25) (layer "F.Cu") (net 2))
 (segment (start 65.1 53.3) (end 65.1 52.1) (width 0.5) (layer "F.Cu") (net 2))
 (via (at 61.4 52.6) (size 0.6) (drill 0.3) (layers "F.Cu" "B.Cu") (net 2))
 (via (at 63.3 58.8) (size 0.6) (drill 0.3) (layers "F.Cu" "B.Cu") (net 2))
 (via (at 63.1 52.1) (size 0.6) (drill 0.3) (layers "F.Cu" "B.Cu") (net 2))
 (via (at 65.1 52.1) (size 0.6) (drill 0.3) (layers "F.Cu" "B.Cu") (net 2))
 (via (at 60.9 51.4) (size 0.6) (drill 0.3) (layers "F.Cu" "B.Cu") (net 2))
 (via (at 67.7 51.1) (size 0.6) (drill 0.3) (layers "F.Cu" "B.Cu") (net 2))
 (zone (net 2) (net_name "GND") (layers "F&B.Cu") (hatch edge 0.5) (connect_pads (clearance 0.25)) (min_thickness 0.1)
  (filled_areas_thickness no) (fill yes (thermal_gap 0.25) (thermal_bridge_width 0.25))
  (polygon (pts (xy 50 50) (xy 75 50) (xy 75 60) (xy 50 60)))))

